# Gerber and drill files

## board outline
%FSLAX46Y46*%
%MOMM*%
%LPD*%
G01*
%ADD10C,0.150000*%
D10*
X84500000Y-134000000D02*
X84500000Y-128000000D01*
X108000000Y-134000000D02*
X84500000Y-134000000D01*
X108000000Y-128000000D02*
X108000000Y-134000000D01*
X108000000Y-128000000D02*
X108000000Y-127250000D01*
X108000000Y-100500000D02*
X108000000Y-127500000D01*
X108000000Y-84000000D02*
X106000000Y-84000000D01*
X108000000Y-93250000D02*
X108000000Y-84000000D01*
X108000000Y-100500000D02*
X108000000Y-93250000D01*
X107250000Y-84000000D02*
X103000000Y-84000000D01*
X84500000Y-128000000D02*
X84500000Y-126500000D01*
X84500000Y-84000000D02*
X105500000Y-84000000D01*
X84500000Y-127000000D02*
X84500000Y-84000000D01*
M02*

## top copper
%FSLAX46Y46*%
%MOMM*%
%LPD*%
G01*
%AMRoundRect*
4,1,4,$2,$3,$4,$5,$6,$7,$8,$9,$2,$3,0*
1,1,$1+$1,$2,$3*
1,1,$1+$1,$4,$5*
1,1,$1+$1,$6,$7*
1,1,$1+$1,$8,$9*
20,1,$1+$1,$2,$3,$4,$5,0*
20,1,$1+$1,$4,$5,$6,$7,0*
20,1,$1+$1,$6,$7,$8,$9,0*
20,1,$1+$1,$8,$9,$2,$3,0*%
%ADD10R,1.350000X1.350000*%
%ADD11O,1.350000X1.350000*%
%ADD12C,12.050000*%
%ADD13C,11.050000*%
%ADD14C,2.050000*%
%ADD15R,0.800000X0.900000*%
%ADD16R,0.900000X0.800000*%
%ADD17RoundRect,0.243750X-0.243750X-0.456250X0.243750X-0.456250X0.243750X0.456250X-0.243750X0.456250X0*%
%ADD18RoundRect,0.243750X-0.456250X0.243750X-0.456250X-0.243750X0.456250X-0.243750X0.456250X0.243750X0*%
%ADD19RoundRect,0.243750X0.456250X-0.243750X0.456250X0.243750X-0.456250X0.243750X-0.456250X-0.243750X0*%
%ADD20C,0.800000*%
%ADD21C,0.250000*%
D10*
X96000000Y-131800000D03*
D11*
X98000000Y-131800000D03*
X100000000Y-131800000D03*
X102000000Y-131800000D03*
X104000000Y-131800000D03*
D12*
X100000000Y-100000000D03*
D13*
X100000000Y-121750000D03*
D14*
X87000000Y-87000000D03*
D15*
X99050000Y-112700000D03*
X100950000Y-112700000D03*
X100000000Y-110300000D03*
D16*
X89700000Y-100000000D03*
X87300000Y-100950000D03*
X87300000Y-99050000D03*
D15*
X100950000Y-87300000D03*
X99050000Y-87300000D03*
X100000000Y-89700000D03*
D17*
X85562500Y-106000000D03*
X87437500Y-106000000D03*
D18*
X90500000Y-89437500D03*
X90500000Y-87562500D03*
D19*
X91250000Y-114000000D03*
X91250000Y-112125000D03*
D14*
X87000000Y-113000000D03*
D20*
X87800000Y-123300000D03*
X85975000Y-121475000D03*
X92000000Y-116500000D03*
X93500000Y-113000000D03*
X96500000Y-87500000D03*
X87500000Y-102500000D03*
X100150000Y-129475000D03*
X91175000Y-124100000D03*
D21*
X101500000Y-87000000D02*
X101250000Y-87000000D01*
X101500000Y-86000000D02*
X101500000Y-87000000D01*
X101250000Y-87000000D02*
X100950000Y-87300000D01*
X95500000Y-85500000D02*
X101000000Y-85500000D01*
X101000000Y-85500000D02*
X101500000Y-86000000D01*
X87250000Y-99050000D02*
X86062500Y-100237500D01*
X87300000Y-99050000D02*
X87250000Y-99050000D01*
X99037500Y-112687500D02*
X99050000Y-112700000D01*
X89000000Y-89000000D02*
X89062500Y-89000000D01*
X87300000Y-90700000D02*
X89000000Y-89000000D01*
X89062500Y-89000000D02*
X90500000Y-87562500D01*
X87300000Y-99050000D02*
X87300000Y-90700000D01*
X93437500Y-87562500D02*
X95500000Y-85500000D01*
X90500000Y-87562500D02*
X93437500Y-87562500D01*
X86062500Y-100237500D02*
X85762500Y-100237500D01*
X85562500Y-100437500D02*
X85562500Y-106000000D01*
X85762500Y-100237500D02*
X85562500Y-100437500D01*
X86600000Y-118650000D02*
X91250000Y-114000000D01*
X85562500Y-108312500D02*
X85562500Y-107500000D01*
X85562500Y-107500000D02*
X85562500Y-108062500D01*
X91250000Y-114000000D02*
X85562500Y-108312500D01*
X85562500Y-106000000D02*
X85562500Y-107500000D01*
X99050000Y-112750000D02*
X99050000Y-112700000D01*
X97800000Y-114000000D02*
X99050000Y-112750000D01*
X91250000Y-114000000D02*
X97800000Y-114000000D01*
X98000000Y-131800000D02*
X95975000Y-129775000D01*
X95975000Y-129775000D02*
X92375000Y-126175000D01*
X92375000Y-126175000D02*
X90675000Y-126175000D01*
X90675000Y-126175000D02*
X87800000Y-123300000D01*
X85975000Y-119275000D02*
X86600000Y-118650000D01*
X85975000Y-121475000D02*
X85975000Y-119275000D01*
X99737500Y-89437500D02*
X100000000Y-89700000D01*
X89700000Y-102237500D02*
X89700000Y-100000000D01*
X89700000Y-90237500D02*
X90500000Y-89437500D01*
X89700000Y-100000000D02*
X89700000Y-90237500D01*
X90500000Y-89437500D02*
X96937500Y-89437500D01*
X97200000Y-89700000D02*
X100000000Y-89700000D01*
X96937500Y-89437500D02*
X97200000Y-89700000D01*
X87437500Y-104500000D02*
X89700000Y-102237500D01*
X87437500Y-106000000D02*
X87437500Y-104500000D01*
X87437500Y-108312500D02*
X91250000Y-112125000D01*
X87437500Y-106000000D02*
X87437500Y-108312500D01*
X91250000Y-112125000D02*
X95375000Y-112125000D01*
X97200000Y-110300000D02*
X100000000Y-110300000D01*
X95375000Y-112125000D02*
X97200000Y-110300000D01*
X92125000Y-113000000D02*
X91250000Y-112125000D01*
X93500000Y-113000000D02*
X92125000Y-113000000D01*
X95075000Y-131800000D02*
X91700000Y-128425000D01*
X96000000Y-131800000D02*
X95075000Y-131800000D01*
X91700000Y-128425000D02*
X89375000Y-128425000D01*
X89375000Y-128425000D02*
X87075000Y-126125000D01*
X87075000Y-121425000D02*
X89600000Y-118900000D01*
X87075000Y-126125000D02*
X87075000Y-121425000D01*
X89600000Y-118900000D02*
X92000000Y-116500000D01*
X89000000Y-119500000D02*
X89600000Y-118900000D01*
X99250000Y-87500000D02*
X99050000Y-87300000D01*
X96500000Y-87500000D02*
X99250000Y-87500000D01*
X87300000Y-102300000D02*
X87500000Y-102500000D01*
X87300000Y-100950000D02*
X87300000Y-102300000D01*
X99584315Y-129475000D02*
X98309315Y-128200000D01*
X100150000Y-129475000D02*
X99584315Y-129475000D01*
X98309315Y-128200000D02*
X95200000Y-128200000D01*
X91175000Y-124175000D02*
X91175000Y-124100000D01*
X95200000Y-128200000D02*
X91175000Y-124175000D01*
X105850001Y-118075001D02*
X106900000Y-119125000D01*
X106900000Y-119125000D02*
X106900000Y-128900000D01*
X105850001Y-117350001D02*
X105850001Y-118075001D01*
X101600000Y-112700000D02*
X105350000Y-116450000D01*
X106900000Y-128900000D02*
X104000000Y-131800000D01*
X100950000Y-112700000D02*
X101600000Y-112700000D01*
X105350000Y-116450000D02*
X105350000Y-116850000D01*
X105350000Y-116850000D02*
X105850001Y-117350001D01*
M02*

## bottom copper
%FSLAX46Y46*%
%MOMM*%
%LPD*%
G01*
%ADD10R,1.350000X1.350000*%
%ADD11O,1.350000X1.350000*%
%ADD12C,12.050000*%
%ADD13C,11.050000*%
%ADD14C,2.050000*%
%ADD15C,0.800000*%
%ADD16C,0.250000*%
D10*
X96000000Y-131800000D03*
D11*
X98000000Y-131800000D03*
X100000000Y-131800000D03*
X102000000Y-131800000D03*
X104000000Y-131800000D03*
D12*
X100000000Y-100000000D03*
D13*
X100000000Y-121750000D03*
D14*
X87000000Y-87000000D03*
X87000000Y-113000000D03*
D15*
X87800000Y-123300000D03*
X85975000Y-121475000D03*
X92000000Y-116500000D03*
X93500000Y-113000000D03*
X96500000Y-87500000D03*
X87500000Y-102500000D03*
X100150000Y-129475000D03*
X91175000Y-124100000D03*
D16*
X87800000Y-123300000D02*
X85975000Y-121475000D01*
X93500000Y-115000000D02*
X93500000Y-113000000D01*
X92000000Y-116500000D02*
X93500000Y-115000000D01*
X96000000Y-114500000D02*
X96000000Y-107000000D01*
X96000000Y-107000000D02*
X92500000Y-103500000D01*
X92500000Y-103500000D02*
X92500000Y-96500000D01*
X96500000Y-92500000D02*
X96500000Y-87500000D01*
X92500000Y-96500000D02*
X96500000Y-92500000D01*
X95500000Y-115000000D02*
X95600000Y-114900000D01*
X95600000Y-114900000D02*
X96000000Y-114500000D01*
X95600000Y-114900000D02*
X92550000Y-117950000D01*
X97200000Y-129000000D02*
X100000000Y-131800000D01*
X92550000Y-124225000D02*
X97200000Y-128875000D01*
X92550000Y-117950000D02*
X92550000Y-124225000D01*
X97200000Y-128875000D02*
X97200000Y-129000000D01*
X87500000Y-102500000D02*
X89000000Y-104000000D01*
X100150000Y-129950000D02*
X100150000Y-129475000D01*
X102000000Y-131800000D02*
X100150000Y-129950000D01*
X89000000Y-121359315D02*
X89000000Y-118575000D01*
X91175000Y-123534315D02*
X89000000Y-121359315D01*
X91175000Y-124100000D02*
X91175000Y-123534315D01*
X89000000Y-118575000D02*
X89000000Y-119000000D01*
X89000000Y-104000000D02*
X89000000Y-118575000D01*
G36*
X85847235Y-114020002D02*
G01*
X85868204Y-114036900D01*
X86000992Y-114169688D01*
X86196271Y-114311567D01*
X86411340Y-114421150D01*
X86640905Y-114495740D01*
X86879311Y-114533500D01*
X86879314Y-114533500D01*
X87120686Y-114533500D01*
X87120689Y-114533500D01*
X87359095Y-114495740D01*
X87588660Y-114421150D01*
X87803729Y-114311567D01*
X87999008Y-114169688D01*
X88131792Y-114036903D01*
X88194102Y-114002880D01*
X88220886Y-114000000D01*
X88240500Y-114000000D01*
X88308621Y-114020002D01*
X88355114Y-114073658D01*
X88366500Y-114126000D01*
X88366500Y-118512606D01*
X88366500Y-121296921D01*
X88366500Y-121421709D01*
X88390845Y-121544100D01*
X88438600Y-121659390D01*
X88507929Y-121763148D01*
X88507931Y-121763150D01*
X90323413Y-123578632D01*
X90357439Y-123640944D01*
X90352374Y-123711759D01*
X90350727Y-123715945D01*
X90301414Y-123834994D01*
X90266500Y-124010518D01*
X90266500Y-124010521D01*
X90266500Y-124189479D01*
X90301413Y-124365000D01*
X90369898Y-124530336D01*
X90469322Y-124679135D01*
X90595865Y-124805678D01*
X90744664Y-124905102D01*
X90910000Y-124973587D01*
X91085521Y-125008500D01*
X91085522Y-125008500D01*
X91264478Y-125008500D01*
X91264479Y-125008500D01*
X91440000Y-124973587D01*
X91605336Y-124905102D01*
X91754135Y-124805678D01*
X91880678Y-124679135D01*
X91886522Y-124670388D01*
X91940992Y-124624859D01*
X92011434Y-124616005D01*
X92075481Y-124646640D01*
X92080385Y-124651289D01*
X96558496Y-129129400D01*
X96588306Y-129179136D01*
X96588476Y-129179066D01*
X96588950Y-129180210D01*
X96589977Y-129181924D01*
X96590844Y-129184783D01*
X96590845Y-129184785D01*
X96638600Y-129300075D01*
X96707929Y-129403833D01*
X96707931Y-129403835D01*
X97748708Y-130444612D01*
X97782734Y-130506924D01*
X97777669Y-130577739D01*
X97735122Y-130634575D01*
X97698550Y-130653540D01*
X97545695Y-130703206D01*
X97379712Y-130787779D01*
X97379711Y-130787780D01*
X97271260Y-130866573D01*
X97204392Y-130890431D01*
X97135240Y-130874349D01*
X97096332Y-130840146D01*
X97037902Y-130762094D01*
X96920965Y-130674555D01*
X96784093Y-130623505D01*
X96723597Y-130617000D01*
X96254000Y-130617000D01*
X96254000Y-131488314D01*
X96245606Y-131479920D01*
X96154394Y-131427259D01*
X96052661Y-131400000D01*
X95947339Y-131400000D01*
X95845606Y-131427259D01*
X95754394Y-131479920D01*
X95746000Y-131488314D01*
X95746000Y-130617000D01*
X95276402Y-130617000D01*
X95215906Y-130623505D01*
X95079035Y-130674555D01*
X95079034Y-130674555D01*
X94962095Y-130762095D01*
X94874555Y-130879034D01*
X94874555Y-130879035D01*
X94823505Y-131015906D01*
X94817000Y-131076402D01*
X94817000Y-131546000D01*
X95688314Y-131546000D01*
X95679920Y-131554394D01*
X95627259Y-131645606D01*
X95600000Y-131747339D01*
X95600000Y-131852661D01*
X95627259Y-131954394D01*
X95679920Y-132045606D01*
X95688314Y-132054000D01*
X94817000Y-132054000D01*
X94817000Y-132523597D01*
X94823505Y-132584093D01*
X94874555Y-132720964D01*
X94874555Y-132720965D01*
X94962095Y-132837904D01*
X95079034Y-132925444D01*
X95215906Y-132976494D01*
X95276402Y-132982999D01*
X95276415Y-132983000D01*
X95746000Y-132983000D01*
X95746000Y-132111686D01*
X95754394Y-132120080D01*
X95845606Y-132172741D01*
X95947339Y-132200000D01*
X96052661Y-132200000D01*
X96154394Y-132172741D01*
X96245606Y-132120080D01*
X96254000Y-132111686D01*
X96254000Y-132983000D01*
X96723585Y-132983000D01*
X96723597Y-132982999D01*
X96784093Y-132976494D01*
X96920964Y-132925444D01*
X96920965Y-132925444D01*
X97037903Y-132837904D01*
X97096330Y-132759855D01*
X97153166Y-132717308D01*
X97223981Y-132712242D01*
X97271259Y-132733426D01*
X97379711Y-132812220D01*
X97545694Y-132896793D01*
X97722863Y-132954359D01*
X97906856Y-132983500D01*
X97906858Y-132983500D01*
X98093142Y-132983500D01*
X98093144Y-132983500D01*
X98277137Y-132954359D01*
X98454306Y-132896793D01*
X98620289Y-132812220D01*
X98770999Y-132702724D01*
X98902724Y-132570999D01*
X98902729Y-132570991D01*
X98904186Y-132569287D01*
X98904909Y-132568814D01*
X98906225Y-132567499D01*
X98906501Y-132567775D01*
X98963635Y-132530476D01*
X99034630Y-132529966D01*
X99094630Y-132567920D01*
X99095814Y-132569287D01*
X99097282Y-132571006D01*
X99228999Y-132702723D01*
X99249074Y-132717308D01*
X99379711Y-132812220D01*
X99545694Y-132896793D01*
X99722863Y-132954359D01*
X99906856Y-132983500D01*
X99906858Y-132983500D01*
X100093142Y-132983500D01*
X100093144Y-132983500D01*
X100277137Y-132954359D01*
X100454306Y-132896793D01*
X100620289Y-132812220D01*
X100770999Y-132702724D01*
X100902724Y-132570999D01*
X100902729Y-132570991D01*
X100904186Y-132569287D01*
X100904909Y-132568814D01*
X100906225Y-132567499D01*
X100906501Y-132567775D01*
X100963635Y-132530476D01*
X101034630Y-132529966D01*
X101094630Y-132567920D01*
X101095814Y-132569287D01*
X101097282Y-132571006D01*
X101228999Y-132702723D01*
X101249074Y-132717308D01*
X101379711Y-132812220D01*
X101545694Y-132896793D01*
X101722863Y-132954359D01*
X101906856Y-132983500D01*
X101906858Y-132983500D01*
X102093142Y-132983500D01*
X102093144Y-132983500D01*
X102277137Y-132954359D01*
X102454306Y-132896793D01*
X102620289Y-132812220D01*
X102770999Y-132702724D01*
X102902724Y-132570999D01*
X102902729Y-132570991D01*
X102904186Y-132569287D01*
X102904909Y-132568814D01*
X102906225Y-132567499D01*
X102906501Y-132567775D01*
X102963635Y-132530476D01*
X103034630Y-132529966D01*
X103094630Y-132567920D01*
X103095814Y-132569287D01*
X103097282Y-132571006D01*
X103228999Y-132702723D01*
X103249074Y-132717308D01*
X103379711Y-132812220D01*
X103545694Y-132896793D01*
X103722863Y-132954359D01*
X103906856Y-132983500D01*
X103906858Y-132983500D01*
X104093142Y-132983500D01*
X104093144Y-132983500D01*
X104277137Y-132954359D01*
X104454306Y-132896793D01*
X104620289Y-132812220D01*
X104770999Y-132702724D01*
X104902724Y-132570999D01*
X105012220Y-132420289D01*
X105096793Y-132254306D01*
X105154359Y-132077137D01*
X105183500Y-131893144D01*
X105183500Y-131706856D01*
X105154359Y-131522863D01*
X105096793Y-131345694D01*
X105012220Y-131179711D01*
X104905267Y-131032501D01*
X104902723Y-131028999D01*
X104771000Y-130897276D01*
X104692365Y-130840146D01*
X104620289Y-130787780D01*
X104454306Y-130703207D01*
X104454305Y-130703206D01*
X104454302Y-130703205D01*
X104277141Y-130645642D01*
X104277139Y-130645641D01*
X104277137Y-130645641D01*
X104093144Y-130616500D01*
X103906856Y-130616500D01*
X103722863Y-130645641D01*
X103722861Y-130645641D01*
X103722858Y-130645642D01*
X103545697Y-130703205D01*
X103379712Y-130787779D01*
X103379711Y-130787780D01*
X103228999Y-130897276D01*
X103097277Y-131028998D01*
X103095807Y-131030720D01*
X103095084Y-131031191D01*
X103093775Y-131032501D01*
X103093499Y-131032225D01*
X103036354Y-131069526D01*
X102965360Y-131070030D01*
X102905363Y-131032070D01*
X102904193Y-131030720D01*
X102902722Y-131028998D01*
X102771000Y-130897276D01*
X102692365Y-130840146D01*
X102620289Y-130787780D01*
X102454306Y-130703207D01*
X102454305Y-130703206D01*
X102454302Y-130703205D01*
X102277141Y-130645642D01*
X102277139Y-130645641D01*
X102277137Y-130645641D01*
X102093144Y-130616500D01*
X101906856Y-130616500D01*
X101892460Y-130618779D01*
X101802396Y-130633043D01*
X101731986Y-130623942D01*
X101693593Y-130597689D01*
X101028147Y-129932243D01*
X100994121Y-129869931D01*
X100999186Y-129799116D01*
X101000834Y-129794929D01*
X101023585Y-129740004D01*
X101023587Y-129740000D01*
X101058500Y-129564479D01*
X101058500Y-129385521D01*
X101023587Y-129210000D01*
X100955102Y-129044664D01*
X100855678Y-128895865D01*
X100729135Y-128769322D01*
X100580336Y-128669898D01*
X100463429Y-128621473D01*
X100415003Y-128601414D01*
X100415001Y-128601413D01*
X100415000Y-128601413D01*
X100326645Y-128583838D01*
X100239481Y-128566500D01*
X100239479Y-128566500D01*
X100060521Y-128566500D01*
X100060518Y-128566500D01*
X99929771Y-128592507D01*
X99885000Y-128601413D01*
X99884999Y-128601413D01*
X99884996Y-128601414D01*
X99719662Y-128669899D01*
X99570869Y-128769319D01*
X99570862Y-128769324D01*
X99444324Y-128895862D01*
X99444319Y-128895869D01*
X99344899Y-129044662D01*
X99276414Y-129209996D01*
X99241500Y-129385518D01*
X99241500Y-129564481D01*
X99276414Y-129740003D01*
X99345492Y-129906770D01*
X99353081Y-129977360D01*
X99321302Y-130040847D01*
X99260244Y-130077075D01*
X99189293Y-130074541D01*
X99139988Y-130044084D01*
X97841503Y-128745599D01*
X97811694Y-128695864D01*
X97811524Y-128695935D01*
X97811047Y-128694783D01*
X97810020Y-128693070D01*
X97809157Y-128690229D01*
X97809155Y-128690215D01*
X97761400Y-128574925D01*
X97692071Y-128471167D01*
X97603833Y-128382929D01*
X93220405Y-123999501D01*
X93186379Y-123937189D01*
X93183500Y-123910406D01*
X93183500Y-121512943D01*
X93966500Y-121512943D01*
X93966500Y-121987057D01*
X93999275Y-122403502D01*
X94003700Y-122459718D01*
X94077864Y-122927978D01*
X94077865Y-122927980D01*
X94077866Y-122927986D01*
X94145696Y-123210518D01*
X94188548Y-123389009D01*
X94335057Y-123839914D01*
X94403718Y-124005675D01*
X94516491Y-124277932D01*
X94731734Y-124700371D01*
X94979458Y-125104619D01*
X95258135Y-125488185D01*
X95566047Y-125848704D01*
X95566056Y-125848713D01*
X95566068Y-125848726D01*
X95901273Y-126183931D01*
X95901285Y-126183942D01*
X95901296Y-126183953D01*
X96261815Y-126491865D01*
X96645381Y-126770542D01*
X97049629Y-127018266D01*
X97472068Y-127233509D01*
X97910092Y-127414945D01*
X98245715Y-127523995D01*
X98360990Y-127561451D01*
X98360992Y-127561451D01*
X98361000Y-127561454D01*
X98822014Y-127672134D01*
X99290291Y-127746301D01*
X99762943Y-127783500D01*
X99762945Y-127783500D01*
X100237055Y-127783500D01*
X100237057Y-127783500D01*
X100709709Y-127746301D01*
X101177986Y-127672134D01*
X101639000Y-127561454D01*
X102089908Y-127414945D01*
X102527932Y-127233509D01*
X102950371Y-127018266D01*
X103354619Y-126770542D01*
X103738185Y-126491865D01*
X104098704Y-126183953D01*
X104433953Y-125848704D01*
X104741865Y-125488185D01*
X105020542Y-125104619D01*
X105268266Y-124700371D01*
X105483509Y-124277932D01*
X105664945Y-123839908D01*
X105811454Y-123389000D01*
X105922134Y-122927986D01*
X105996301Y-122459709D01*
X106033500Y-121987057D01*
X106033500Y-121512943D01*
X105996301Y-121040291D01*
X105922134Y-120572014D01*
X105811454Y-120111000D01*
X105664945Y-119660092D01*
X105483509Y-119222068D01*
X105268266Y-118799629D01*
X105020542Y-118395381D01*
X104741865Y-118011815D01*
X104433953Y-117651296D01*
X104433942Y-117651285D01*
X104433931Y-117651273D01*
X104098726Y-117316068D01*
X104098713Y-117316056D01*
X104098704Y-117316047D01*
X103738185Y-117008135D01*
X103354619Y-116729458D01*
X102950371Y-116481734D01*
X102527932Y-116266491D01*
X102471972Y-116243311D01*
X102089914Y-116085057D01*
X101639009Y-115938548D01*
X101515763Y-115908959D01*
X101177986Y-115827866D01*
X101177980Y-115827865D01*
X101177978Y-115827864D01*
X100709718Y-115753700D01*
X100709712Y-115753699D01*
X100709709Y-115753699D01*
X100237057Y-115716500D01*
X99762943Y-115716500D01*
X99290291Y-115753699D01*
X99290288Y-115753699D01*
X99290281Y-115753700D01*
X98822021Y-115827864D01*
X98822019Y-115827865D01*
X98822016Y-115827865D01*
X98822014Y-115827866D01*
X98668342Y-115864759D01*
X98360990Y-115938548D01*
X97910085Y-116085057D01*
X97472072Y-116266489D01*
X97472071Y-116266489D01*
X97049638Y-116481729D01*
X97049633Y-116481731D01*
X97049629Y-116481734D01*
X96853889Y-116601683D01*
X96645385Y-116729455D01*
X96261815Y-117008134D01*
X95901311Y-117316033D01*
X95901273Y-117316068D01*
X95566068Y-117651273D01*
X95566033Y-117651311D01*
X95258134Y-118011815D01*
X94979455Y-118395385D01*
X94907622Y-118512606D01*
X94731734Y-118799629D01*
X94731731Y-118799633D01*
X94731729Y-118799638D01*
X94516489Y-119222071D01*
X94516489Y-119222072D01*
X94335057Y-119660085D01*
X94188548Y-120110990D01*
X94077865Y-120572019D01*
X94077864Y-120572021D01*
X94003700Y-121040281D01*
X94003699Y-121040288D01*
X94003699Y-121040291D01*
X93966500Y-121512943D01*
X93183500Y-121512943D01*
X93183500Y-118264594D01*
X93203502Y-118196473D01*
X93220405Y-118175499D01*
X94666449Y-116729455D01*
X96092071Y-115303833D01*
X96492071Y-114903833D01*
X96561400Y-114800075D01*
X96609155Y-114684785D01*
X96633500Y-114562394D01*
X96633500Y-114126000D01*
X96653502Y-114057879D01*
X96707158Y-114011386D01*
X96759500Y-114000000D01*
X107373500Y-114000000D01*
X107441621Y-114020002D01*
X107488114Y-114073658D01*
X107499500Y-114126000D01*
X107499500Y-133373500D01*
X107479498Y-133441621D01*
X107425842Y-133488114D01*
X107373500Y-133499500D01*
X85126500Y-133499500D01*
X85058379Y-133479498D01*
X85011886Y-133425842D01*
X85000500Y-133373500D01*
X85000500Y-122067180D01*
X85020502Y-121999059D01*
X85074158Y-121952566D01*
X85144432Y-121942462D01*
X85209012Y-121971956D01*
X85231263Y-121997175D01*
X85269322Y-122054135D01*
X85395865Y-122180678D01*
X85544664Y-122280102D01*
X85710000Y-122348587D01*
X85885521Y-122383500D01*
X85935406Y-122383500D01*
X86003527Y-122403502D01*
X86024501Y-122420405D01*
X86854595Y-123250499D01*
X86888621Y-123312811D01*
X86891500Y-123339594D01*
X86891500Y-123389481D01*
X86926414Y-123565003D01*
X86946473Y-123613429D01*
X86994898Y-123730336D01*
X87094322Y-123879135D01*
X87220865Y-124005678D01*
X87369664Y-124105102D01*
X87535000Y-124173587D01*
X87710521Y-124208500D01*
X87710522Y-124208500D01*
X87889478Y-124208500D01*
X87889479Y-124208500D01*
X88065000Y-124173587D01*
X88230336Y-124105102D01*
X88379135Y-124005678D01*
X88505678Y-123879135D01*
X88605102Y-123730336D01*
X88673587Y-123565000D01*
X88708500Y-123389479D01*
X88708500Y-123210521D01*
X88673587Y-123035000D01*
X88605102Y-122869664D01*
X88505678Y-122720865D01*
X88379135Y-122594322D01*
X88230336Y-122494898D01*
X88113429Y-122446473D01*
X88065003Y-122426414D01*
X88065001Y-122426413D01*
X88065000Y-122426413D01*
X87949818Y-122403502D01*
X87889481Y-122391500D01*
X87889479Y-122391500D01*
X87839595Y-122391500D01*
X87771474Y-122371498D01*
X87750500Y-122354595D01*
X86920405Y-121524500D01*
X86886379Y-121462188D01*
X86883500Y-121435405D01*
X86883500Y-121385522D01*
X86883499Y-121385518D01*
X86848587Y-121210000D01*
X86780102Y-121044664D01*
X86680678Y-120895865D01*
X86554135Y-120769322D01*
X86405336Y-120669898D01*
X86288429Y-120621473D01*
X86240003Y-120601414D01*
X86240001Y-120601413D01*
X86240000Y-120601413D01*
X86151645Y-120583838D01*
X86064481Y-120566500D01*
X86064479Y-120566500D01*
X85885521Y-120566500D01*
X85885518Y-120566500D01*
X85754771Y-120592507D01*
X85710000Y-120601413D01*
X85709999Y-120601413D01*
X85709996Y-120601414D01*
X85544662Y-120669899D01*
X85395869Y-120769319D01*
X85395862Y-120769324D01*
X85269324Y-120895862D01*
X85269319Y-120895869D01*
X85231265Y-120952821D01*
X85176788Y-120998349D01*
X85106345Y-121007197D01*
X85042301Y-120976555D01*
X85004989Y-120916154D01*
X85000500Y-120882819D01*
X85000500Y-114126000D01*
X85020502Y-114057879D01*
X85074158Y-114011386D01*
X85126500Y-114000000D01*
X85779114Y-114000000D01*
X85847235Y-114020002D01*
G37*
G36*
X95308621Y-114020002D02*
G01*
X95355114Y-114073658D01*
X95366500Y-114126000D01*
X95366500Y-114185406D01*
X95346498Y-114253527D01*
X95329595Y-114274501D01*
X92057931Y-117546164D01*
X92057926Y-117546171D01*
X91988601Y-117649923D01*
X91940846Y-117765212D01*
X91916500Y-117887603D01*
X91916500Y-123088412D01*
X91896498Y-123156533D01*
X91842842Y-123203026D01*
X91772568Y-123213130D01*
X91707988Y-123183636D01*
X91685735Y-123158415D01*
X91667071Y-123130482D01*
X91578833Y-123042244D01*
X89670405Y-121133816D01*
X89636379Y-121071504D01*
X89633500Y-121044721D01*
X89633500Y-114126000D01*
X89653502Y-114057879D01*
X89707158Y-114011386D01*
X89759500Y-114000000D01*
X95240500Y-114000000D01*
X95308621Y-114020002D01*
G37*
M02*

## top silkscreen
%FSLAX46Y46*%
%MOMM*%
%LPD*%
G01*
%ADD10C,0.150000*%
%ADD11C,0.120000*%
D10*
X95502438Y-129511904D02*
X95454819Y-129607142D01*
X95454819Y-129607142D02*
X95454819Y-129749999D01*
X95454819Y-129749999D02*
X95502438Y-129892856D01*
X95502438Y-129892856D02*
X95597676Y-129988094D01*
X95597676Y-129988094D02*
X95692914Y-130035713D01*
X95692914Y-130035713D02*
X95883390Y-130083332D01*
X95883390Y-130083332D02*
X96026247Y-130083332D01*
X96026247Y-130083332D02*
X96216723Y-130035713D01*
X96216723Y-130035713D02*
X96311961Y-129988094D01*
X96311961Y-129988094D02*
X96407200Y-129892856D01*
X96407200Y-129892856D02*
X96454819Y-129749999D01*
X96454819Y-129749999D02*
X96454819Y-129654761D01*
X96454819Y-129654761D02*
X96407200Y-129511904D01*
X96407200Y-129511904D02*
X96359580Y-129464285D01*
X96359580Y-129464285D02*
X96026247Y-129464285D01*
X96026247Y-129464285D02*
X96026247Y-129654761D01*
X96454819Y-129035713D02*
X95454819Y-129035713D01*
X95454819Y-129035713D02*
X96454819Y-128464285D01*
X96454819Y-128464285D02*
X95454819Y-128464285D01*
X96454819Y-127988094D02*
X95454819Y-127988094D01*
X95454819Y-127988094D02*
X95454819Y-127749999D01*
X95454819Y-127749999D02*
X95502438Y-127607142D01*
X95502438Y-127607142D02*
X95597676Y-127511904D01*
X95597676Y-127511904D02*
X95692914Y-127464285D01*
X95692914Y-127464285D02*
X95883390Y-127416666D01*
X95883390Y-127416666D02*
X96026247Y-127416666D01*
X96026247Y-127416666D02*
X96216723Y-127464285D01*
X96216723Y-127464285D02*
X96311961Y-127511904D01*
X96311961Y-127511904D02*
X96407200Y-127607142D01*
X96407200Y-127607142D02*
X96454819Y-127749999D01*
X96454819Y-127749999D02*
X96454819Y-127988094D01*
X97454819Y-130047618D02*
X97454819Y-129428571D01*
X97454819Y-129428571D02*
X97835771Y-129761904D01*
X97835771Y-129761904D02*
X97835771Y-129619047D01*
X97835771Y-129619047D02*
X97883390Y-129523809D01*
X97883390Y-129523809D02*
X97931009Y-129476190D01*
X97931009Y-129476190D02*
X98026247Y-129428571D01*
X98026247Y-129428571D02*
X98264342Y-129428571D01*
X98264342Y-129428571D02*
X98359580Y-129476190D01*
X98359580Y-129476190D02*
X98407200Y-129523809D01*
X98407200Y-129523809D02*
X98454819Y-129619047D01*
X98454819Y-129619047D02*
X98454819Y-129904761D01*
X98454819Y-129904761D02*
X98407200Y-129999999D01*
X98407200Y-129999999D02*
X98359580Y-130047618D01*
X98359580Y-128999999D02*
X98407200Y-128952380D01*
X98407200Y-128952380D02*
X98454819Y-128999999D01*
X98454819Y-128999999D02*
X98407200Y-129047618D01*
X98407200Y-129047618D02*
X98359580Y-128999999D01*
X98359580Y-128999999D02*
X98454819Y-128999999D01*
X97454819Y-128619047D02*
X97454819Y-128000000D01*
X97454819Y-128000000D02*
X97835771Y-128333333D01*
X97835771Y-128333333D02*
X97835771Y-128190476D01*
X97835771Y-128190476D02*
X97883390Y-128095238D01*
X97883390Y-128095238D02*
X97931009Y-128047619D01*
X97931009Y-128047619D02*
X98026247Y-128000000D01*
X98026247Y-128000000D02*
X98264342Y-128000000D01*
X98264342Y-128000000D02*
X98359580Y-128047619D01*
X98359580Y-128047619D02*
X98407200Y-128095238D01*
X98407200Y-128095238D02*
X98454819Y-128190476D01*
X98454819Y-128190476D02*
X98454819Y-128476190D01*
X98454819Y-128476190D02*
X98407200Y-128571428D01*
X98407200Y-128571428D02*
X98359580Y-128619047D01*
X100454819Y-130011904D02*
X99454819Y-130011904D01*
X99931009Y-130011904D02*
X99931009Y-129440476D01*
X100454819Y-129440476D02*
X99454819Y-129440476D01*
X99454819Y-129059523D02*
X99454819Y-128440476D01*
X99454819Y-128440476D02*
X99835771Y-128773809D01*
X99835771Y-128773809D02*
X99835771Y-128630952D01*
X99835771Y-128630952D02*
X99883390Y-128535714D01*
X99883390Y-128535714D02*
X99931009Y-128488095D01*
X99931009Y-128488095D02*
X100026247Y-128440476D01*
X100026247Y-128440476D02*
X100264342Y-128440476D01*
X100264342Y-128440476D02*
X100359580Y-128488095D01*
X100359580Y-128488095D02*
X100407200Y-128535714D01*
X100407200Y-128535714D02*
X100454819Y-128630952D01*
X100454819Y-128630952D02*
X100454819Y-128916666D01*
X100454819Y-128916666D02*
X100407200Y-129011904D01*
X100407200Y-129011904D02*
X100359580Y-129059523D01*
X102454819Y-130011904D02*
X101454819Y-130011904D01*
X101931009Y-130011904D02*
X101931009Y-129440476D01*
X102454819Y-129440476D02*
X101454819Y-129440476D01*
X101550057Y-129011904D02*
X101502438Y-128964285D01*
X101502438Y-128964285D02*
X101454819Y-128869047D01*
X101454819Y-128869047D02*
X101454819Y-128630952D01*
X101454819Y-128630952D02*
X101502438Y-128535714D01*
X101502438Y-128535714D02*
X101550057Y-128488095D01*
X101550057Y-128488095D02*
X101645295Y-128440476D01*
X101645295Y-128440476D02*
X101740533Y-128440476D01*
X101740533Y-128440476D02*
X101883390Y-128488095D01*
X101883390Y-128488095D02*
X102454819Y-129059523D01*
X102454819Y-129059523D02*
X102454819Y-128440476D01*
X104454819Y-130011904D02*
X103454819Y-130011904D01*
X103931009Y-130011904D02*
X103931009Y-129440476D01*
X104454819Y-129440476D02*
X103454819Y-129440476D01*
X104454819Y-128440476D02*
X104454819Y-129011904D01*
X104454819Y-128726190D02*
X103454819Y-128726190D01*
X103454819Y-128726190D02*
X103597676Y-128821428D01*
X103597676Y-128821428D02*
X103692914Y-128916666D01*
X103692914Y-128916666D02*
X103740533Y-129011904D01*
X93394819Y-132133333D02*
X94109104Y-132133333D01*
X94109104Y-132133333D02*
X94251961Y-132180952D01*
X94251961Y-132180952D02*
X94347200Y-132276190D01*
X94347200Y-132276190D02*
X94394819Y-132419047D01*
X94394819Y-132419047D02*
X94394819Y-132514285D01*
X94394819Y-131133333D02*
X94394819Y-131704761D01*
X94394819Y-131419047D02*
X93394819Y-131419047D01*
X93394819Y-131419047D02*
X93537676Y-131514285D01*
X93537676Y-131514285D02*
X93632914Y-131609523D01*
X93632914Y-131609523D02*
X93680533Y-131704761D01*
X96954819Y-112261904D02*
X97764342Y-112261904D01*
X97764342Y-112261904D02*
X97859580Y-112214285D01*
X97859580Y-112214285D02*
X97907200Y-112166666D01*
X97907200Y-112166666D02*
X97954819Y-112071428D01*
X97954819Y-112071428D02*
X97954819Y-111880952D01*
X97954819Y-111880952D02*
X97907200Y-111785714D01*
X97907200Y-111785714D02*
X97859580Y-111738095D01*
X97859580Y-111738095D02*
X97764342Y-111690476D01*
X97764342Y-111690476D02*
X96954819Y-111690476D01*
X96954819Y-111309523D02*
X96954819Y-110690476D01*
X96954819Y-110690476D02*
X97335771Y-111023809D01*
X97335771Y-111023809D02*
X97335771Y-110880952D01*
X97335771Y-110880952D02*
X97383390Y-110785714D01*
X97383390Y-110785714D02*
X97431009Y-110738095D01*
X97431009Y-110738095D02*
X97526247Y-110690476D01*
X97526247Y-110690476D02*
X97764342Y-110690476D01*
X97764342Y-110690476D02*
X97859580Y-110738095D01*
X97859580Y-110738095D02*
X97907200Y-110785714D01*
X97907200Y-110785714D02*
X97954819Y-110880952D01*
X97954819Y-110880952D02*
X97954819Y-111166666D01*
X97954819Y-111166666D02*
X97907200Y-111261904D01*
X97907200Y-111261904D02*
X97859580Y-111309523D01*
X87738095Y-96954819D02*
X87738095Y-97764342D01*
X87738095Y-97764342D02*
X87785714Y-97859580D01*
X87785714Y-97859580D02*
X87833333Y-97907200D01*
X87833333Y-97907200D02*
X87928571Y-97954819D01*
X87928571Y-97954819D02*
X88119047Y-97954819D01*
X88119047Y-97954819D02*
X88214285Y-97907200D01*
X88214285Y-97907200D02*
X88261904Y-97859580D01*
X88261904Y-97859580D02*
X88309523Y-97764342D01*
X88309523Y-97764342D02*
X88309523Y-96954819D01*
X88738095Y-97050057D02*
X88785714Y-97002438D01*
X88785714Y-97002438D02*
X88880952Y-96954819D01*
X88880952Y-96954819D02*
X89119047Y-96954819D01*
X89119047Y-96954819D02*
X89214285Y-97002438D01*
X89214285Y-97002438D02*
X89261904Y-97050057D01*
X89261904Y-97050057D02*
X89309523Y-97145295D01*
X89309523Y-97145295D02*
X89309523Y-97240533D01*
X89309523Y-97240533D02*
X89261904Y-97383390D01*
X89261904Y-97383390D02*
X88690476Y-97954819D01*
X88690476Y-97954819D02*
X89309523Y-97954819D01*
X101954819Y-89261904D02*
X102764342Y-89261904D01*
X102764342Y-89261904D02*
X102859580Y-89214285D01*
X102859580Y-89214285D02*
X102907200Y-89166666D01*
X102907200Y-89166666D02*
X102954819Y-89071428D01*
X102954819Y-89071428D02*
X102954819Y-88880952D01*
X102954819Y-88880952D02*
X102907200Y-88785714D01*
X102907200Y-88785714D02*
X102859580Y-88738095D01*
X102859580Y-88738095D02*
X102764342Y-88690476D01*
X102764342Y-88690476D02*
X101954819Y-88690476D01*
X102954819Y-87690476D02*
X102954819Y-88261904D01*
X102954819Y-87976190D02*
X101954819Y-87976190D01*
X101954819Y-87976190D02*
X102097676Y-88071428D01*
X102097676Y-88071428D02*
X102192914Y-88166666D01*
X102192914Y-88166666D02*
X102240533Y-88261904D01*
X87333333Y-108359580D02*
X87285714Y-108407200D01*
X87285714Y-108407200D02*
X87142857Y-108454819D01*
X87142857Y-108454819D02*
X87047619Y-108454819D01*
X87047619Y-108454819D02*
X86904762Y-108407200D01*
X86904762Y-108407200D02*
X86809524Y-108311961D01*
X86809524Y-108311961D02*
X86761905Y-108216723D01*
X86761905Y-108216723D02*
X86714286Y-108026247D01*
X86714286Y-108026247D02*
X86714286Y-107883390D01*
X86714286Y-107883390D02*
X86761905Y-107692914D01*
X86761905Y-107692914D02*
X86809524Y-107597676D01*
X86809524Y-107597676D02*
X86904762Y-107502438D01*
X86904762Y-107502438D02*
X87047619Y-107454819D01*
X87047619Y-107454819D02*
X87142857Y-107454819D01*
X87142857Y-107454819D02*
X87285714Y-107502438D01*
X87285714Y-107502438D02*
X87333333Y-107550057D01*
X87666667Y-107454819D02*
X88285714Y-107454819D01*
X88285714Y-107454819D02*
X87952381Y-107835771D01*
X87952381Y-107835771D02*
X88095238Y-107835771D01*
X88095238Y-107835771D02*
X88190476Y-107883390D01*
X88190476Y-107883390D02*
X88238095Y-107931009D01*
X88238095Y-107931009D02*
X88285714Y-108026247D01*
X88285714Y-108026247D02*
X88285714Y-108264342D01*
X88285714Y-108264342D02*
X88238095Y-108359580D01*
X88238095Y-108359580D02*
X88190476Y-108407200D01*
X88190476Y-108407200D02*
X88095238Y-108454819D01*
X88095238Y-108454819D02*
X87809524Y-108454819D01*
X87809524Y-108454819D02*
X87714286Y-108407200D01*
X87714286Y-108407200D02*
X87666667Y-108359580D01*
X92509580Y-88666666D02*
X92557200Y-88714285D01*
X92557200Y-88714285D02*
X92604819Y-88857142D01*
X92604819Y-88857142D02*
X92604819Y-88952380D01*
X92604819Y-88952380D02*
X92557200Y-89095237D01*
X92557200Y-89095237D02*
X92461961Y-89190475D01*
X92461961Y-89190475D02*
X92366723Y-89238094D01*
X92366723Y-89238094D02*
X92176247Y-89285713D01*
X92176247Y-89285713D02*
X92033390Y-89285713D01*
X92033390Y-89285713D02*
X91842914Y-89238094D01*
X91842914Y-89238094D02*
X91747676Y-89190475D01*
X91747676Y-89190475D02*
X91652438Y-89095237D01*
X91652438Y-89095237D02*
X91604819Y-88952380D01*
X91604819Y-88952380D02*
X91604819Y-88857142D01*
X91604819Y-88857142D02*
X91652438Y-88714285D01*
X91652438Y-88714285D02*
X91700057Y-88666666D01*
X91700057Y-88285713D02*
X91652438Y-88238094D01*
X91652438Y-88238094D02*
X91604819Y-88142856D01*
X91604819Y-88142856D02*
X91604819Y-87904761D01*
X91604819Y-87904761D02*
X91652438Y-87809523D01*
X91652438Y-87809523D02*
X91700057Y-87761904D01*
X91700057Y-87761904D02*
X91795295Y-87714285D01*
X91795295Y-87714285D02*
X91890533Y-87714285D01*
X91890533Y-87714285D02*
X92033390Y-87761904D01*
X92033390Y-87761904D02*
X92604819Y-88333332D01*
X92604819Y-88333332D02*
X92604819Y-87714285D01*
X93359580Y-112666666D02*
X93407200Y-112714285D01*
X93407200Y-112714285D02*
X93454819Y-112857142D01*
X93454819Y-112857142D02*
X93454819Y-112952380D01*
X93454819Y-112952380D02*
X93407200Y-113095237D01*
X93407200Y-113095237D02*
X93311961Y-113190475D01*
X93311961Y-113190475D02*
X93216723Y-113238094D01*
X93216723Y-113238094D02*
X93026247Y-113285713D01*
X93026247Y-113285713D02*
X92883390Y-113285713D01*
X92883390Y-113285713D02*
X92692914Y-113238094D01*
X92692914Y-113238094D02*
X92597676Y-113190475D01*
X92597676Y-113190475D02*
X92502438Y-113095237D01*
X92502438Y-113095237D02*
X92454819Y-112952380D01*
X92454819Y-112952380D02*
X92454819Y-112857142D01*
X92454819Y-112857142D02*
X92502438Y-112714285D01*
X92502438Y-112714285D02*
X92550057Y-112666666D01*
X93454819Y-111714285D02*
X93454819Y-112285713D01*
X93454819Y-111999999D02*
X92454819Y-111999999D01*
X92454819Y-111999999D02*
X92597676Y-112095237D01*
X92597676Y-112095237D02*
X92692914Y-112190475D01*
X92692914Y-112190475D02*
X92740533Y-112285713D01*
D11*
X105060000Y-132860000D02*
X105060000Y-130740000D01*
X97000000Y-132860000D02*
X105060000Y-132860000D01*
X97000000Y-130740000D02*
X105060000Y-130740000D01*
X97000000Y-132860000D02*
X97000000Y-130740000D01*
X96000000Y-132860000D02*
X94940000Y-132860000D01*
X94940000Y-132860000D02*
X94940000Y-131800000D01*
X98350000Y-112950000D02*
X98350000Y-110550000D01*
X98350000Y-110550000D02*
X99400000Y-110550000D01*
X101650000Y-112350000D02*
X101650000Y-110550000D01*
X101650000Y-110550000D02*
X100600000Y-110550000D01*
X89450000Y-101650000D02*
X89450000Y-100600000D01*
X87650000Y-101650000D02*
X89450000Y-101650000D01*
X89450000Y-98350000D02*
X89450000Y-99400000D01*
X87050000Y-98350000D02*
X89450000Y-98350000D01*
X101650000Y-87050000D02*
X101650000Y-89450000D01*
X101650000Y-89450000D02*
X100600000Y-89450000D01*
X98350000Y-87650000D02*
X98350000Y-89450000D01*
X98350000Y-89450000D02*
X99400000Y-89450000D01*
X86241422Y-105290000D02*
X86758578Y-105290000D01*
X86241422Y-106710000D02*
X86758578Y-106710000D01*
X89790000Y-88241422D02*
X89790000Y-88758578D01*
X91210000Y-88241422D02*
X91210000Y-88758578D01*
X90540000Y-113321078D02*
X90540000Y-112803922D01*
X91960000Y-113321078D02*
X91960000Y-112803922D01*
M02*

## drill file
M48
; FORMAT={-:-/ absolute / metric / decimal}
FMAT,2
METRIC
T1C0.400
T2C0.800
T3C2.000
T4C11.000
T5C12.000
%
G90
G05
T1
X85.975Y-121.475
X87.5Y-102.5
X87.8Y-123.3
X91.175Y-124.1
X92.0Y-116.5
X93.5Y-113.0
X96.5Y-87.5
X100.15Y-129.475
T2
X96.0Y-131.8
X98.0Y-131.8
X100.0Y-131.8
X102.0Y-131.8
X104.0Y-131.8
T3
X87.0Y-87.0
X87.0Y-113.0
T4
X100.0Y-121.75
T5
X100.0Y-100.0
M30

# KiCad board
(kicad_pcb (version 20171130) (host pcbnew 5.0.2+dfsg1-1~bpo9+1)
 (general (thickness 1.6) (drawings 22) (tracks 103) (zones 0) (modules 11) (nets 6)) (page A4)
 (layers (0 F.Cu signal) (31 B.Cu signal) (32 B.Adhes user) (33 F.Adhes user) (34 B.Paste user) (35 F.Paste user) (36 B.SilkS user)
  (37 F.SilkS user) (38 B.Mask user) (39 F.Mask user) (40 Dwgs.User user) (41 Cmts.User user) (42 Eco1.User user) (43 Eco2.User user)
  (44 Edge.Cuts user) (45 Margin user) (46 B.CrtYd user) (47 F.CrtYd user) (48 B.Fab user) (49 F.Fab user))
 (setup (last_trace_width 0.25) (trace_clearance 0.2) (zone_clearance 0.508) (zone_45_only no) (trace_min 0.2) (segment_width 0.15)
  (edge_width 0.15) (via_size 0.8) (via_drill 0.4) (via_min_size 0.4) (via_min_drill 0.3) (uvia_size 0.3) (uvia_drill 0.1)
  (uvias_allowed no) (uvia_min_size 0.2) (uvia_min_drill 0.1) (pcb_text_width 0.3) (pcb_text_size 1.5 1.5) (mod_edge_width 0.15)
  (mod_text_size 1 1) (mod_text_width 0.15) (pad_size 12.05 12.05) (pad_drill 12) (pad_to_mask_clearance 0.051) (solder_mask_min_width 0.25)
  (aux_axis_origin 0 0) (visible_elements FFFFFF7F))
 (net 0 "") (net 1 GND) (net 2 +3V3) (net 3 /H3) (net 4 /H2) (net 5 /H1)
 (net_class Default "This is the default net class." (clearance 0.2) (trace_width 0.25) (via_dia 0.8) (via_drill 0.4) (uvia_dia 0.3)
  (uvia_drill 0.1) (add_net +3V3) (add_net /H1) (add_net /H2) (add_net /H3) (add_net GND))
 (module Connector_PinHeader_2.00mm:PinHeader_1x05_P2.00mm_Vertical (layer F.Cu) (at 96 131.8 90)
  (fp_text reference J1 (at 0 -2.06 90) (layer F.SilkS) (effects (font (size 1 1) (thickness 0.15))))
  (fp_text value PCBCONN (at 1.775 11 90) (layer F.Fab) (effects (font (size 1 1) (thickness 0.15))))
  (fp_line (start -1.06 9.06) (end 1.06 9.06) (layer F.SilkS) (width 0.12))
  (fp_line (start -1.06 1) (end -1.06 9.06) (layer F.SilkS) (width 0.12))
  (fp_line (start 1.06 1) (end 1.06 9.06) (layer F.SilkS) (width 0.12))
  (fp_line (start -1.06 1) (end 1.06 1) (layer F.SilkS) (width 0.12))
  (fp_line (start -1.06 0) (end -1.06 -1.06) (layer F.SilkS) (width 0.12))
  (fp_line (start -1.06 -1.06) (end 0 -1.06) (layer F.SilkS) (width 0.12))
  (pad 1 thru_hole rect (at 0 0 90) (size 1.35 1.35) (drill 0.8) (layers *.Cu *.Mask) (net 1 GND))
  (pad 2 thru_hole oval (at 0 2 90) (size 1.35 1.35) (drill 0.8) (layers *.Cu *.Mask) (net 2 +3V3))
  (pad 3 thru_hole oval (at 0 4 90) (size 1.35 1.35) (drill 0.8) (layers *.Cu *.Mask) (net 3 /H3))
  (pad 4 thru_hole oval (at 0 6 90) (size 1.35 1.35) (drill 0.8) (layers *.Cu *.Mask) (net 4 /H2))
  (pad 5 thru_hole oval (at 0 8 90) (size 1.35 1.35) (drill 0.8) (layers *.Cu *.Mask) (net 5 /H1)))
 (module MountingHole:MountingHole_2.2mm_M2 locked (layer F.Cu) (at 100 100)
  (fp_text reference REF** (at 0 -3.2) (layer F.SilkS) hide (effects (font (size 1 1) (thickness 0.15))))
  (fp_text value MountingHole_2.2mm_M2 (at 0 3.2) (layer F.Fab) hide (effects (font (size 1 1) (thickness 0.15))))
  (pad "" np_thru_hole circle (at 0 0) (size 12.05 12.05) (drill 12) (layers *.Cu *.Mask)))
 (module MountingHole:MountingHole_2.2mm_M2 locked (layer F.Cu) (at 100 121.75)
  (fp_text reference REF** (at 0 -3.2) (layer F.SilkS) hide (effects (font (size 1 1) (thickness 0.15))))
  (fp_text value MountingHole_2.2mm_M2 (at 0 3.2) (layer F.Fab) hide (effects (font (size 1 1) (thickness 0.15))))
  (pad "" np_thru_hole circle (at 0 0) (size 11.05 11.05) (drill 11) (layers *.Cu *.Mask)))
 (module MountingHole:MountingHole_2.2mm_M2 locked (layer F.Cu) (at 87 87)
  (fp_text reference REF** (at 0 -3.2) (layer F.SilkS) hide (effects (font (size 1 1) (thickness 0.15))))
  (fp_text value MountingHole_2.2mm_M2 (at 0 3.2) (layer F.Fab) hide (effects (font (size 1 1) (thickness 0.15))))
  (pad "" np_thru_hole circle (at 0 0) (size 2.05 2.05) (drill 2) (layers *.Cu *.Mask)))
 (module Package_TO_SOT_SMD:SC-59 (layer F.Cu) (at 100 111.5 90)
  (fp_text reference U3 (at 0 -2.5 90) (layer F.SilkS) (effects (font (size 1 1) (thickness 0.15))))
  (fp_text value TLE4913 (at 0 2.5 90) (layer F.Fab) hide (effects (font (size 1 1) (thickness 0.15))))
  (fp_line (start -1.45 -1.65) (end 0.95 -1.65) (layer F.SilkS) (width 0.12))
  (fp_line (start 0.95 -1.65) (end 0.95 -0.6) (layer F.SilkS) (width 0.12))
  (fp_line (start -0.85 1.65) (end 0.95 1.65) (layer F.SilkS) (width 0.12))
  (fp_line (start 0.95 1.65) (end 0.95 0.6) (layer F.SilkS) (width 0.12))
  (pad 1 smd rect (at -1.2 -0.95 90) (size 0.9 0.8) (layers F.Cu F.Paste F.Mask) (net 2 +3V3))
  (pad 2 smd rect (at -1.2 0.95 90) (size 0.9 0.8) (layers F.Cu F.Paste F.Mask) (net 5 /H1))
  (pad 3 smd rect (at 1.2 0 90) (size 0.9 0.8) (layers F.Cu F.Paste F.Mask) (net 1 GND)))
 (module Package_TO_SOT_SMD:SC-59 (layer F.Cu) (at 88.5 100)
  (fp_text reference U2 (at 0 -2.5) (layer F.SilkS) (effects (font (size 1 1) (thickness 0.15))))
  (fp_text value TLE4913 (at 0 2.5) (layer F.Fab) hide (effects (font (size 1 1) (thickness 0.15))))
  (fp_line (start 0.95 1.65) (end 0.95 0.6) (layer F.SilkS) (width 0.12))
  (fp_line (start -0.85 1.65) (end 0.95 1.65) (layer F.SilkS) (width 0.12))
  (fp_line (start 0.95 -1.65) (end 0.95 -0.6) (layer F.SilkS) (width 0.12))
  (fp_line (start -1.45 -1.65) (end 0.95 -1.65) (layer F.SilkS) (width 0.12))
  (pad 3 smd rect (at 1.2 0) (size 0.9 0.8) (layers F.Cu F.Paste F.Mask) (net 1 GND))
  (pad 2 smd rect (at -1.2 0.95) (size 0.9 0.8) (layers F.Cu F.Paste F.Mask) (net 4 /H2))
  (pad 1 smd rect (at -1.2 -0.95) (size 0.9 0.8) (layers F.Cu F.Paste F.Mask) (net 2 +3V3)))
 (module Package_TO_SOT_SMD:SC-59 (layer F.Cu) (at 100 88.5 270)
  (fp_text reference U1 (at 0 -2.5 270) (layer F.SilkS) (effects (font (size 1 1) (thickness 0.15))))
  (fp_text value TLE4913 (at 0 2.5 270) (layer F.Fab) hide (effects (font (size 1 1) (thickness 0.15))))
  (fp_line (start -1.45 -1.65) (end 0.95 -1.65) (layer F.SilkS) (width 0.12))
  (fp_line (start 0.95 -1.65) (end 0.95 -0.6) (layer F.SilkS) (width 0.12))
  (fp_line (start -0.85 1.65) (end 0.95 1.65) (layer F.SilkS) (width 0.12))
  (fp_line (start 0.95 1.65) (end 0.95 0.6) (layer F.SilkS) (width 0.12))
  (pad 1 smd rect (at -1.2 -0.95 270) (size 0.9 0.8) (layers F.Cu F.Paste F.Mask) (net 2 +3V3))
  (pad 2 smd rect (at -1.2 0.95 270) (size 0.9 0.8) (layers F.Cu F.Paste F.Mask) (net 3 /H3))
  (pad 3 smd rect (at 1.2 0 270) (size 0.9 0.8) (layers F.Cu F.Paste F.Mask) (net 1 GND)))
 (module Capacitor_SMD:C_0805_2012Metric (layer F.Cu) (at 86.5 106)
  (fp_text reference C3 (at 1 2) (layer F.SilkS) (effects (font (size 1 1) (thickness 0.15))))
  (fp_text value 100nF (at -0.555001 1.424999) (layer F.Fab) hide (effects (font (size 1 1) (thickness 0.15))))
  (fp_line (start -0.258578 -0.71) (end 0.258578 -0.71) (layer F.SilkS) (width 0.12))
  (fp_line (start -0.258578 0.71) (end 0.258578 0.71) (layer F.SilkS) (width 0.12))
  (pad 1 smd roundrect (at -0.9375 0) (size 0.975 1.4) (layers F.Cu F.Paste F.Mask) (roundrect_rratio 0.25) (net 2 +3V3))
  (pad 2 smd roundrect (at 0.9375 0) (size 0.975 1.4) (layers F.Cu F.Paste F.Mask) (roundrect_rratio 0.25) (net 1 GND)))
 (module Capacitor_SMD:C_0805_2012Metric (layer F.Cu) (at 90.5 88.5 270)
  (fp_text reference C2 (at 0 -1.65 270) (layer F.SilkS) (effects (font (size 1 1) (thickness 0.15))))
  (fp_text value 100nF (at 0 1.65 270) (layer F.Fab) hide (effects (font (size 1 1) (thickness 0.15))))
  (fp_line (start -0.258578 0.71) (end 0.258578 0.71) (layer F.SilkS) (width 0.12))
  (fp_line (start -0.258578 -0.71) (end 0.258578 -0.71) (layer F.SilkS) (width 0.12))
  (pad 2 smd roundrect (at 0.9375 0 270) (size 0.975 1.4) (layers F.Cu F.Paste F.Mask) (roundrect_rratio 0.25) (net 1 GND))
  (pad 1 smd roundrect (at -0.9375 0 270) (size 0.975 1.4) (layers F.Cu F.Paste F.Mask) (roundrect_rratio 0.25) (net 2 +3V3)))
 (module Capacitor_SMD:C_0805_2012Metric (layer F.Cu) (at 91.25 113.0625 90)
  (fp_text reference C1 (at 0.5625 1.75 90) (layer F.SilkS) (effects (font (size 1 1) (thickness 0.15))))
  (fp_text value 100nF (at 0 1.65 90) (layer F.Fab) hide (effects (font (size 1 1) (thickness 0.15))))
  (fp_line (start -0.258578 -0.71) (end 0.258578 -0.71) (layer F.SilkS) (width 0.12))
  (fp_line (start -0.258578 0.71) (end 0.258578 0.71) (layer F.SilkS) (width 0.12))
  (pad 1 smd roundrect (at -0.9375 0 90) (size 0.975 1.4) (layers F.Cu F.Paste F.Mask) (roundrect_rratio 0.25) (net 2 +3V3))
  (pad 2 smd roundrect (at 0.9375 0 90) (size 0.975 1.4) (layers F.Cu F.Paste F.Mask) (roundrect_rratio 0.25) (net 1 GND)))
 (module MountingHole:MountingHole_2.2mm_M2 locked (layer F.Cu) (at 87 113)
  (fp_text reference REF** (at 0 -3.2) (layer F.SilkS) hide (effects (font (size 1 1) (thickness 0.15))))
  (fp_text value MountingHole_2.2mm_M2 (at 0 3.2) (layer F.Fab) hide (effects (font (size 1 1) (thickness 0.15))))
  (pad "" np_thru_hole circle (at 0 0) (size 2.05 2.05) (drill 2) (layers *.Cu *.Mask)))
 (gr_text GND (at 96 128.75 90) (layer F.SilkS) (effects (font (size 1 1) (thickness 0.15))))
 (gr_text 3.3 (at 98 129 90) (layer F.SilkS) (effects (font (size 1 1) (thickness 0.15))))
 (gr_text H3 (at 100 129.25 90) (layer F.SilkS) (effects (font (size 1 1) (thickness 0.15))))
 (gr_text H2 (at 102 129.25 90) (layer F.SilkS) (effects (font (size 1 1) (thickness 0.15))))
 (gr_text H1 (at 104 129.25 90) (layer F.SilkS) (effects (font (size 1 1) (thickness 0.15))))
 (gr_line (start 84.5 134) (end 84.5 128) (layer Edge.Cuts) (width 0.15))
 (gr_line (start 108 134) (end 84.5 134) (layer Edge.Cuts) (width 0.15))
 (gr_line (start 108 128) (end 108 134) (layer Edge.Cuts) (width 0.15))
 (gr_line (start 108 128) (end 108 127.25) (layer Edge.Cuts) (width 0.15))
 (gr_line (start 108 100.5) (end 108 127.5) (layer Edge.Cuts) (width 0.15))
 (gr_line (start 108 84) (end 106 84) (layer Edge.Cuts) (width 0.15))
 (gr_line (start 108 93.25) (end 108 84) (layer Edge.Cuts) (width 0.15))
 (gr_line (start 108 100.5) (end 108 93.25) (layer Edge.Cuts) (width 0.15))
 (gr_line (start 107.25 84) (end 103 84) (layer Edge.Cuts) (width 0.15))
 (gr_line (start 84.5 128) (end 84.5 126.5) (layer Edge.Cuts) (width 0.15))
 (gr_line (start 84.5 84) (end 105.5 84) (layer Edge.Cuts) (width 0.15))
 (gr_line (start 84.5 127) (end 84.5 84) (layer Edge.Cuts) (width 0.15))
 (segment (start 101.5 87) (end 101.25 87) (width 0.25) (layer F.Cu) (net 2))
 (segment (start 101.5 86) (end 101.5 87) (width 0.25) (layer F.Cu) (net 2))
 (segment (start 101.25 87) (end 100.95 87.3) (width 0.25) (layer F.Cu) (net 2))
 (segment (start 95.5 85.5) (end 101 85.5) (width 0.25) (layer F.Cu) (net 2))
 (segment (start 101 85.5) (end 101.5 86) (width 0.25) (layer F.Cu) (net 2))
 (segment (start 87.25 99.05) (end 86.0625 100.2375) (width 0.25) (layer F.Cu) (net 2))
 (segment (start 87.3 99.05) (end 87.25 99.05) (width 0.25) (layer F.Cu) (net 2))
 (segment (start 99.0375 112.6875) (end 99.05 112.7) (width 0.25) (layer F.Cu) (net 2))
 (segment (start 89 89) (end 89.0625 89) (width 0.25) (layer F.Cu) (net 2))
 (segment (start 87.3 90.7) (end 89 89) (width 0.25) (layer F.Cu) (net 2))
 (segment (start 89.0625 89) (end 90.5 87.5625) (width 0.25) (layer F.Cu) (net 2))
 (segment (start 87.3 99.05) (end 87.3 90.7) (width 0.25) (layer F.Cu) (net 2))
 (segment (start 93.4375 87.5625) (end 95.5 85.5) (width 0.25) (layer F.Cu) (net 2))
 (segment (start 90.5 87.5625) (end 93.4375 87.5625) (width 0.25) (layer F.Cu) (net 2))
 (segment (start 86.0625 100.2375) (end 85.7625 100.2375) (width 0.25) (layer F.Cu) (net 2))
 (segment (start 85.5625 100.4375) (end 85.5625 106) (width 0.25) (layer F.Cu) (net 2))
 (segment (start 85.7625 100.2375) (end 85.5625 100.4375) (width 0.25) (layer F.Cu) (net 2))
 (segment (start 86.6 118.65) (end 91.25 114) (width 0.25) (layer F.Cu) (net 2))
 (segment (start 85.5625 108.3125) (end 85.5625 107.5) (width 0.25) (layer F.Cu) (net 2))
 (segment (start 85.5625 107.5) (end 85.5625 108.0625) (width 0.25) (layer F.Cu) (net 2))
 (segment (start 91.25 114) (end 85.5625 108.3125) (width 0.25) (layer F.Cu) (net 2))
 (segment (start 85.5625 106) (end 85.5625 107.5) (width 0.25) (layer F.Cu) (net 2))
 (segment (start 99.05 112.75) (end 99.05 112.7) (width 0.25) (layer F.Cu) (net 2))
 (segment (start 97.8 114) (end 99.05 112.75) (width 0.25) (layer F.Cu) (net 2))
 (segment (start 91.25 114) (end 97.8 114) (width 0.25) (layer F.Cu) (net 2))
 (segment (start 98 131.8) (end 95.975 129.775) (width 0.25) (layer F.Cu) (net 2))
 (segment (start 95.975 129.775) (end 92.375 126.175) (width 0.25) (layer F.Cu) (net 2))
 (segment (start 92.375 126.175) (end 90.675 126.175) (width 0.25) (layer F.Cu) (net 2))
 (via (at 87.8 123.3) (size 0.8) (drill 0.4) (layers F.Cu B.Cu) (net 2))
 (segment (start 90.675 126.175) (end 87.8 123.3) (width 0.25) (layer F.Cu) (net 2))
 (segment (start 87.8 123.3) (end 85.975 121.475) (width 0.25) (layer B.Cu) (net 2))
 (via (at 85.975 121.475) (size 0.8) (drill 0.4) (layers F.Cu B.Cu) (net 2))
 (segment (start 85.975 119.275) (end 86.6 118.65) (width 0.25) (layer F.Cu) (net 2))
 (segment (start 85.975 121.475) (end 85.975 119.275) (width 0.25) (layer F.Cu) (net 2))
 (segment (start 99.7375 89.4375) (end 100 89.7) (width 0.25) (layer F.Cu) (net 1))
 (segment (start 89.7 102.2375) (end 89.7 100) (width 0.25) (layer F.Cu) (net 1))
 (segment (start 89.7 90.2375) (end 90.5 89.4375) (width 0.25) (layer F.Cu) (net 1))
 (segment (start 89.7 100) (end 89.7 90.2375) (width 0.25) (layer F.Cu) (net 1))
 (segment (start 90.5 89.4375) (end 96.9375 89.4375) (width 0.25) (layer F.Cu) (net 1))
 (segment (start 97.2 89.7) (end 100 89.7) (width 0.25) (layer F.Cu) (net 1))
 (segment (start 96.9375 89.4375) (end 97.2 89.7) (width 0.25) (layer F.Cu) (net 1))
 (segment (start 87.4375 104.5) (end 89.7 102.2375) (width 0.25) (layer F.Cu) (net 1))
 (segment (start 87.4375 106) (end 87.4375 104.5) (width 0.25) (layer F.Cu) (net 1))
 (segment (start 87.4375 108.3125) (end 91.25 112.125) (width 0.25) (layer F.Cu) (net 1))
 (segment (start 87.4375 106) (end 87.4375 108.3125) (width 0.25) (layer F.Cu) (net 1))
 (segment (start 91.25 112.125) (end 95.375 112.125) (width 0.25) (layer F.Cu) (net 1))
 (segment (start 97.2 110.3) (end 100 110.3) (width 0.25) (layer F.Cu) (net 1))
 (segment (start 95.375 112.125) (end 97.2 110.3) (width 0.25) (layer F.Cu) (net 1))
 (via (at 92 116.5) (size 0.8) (drill 0.4) (layers F.Cu B.Cu) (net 1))
 (via (at 93.5 113) (size 0.8) (drill 0.4) (layers F.Cu B.Cu) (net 1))
 (segment (start 93.5 115) (end 93.5 113) (width 0.25) (layer B.Cu) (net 1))
 (segment (start 92 116.5) (end 93.5 115) (width 0.25) (layer B.Cu) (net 1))
 (segment (start 92.125 113) (end 91.25 112.125) (width 0.25) (layer F.Cu) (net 1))
 (segment (start 93.5 113) (end 92.125 113) (width 0.25) (layer F.Cu) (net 1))
 (segment (start 95.075 131.8) (end 91.7 128.425) (width 0.25) (layer F.Cu) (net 1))
 (segment (start 96 131.8) (end 95.075 131.8) (width 0.25) (layer F.Cu) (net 1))
 (segment (start 91.7 128.425) (end 89.375 128.425) (width 0.25) (layer F.Cu) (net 1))
 (segment (start 89.375 128.425) (end 87.075 126.125) (width 0.25) (layer F.Cu) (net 1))
 (segment (start 87.075 121.425) (end 89.6 118.9) (width 0.25) (layer F.Cu) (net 1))
 (segment (start 87.075 126.125) (end 87.075 121.425) (width 0.25) (layer F.Cu) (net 1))
 (segment (start 89.6 118.9) (end 92 116.5) (width 0.25) (layer F.Cu) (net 1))
 (segment (start 89 119.5) (end 89.6 118.9) (width 0.25) (layer F.Cu) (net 1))
 (segment (start 96 114.5) (end 96 107) (width 0.25) (layer B.Cu) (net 3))
 (segment (start 96 107) (end 92.5 103.5) (width 0.25) (layer B.Cu) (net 3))
 (segment (start 92.5 103.5) (end 92.5 96.5) (width 0.25) (layer B.Cu) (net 3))
 (via (at 96.5 87.5) (size 0.8) (drill 0.4) (layers F.Cu B.Cu) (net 3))
 (segment (start 96.5 92.5) (end 96.5 87.5) (width 0.25) (layer B.Cu) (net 3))
 (segment (start 92.5 96.5) (end 96.5 92.5) (width 0.25) (layer B.Cu) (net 3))
 (segment (start 99.25 87.5) (end 99.05 87.3) (width 0.25) (layer F.Cu) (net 3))
 (segment (start 96.5 87.5) (end 99.25 87.5) (width 0.25) (layer F.Cu) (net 3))
 (segment (start 95.5 115) (end 95.6 114.9) (width 0.25) (layer B.Cu) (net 3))
 (segment (start 95.6 114.9) (end 96 114.5) (width 0.25) (layer B.Cu) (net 3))
 (segment (start 95.6 114.9) (end 92.55 117.95) (width 0.25) (layer B.Cu) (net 3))
 (segment (start 97.2 129) (end 100 131.8) (width 0.25) (layer B.Cu) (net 3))
 (segment (start 92.55 124.225) (end 97.2 128.875) (width 0.25) (layer B.Cu) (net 3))
 (segment (start 92.55 117.95) (end 92.55 124.225) (width 0.25) (layer B.Cu) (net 3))
 (segment (start 97.2 128.875) (end 97.2 129) (width 0.25) (layer B.Cu) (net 3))
 (via (at 87.5 102.5) (size 0.8) (drill 0.4) (layers F.Cu B.Cu) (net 4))
 (segment (start 87.3 102.3) (end 87.5 102.5) (width 0.25) (layer F.Cu) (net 4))
 (segment (start 87.3 100.95) (end 87.3 102.3) (width 0.25) (layer F.Cu) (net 4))
 (segment (start 87.5 102.5) (end 89 104) (width 0.25) (layer B.Cu) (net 4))
 (via (at 100.15 129.475) (size 0.8) (drill 0.4) (layers F.Cu B.Cu) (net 4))
 (segment (start 100.15 129.95) (end 100.15 129.475) (width 0.25) (layer B.Cu) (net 4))
 (segment (start 102 131.8) (end 100.15 129.95) (width 0.25) (layer B.Cu) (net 4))
 (segment (start 99.584315 129.475) (end 98.309315 128.2) (width 0.25) (layer F.Cu) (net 4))
 (segment (start 100.15 129.475) (end 99.584315 129.475) (width 0.25) (layer F.Cu) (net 4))
 (segment (start 98.309315 128.2) (end 95.2 128.2) (width 0.25) (layer F.Cu) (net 4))
 (via (at 91.175 124.1) (size 0.8) (drill 0.4) (layers F.Cu B.Cu) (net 4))
 (segment (start 91.175 124.175) (end 91.175 124.1) (width 0.25) (layer F.Cu) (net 4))
 (segment (start 95.2 128.2) (end 91.175 124.175) (width 0.25) (layer F.Cu) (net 4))
 (segment (start 89 121.359315) (end 89 118.575) (width 0.25) (layer B.Cu) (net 4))
 (segment (start 91.175 123.534315) (end 89 121.359315) (width 0.25) (layer B.Cu) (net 4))
 (segment (start 91.175 124.1) (end 91.175 123.534315) (width 0.25) (layer B.Cu) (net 4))
 (segment (start 89 118.575) (end 89 119) (width 0.25) (layer B.Cu) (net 4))
 (segment (start 89 104) (end 89 118.575) (width 0.25) (layer B.Cu) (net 4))
 (segment (start 105.850001 118.075001) (end 106.9 119.125) (width 0.25) (layer F.Cu) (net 5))
 (segment (start 106.9 119.125) (end 106.9 128.9) (width 0.25) (layer F.Cu) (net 5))
 (segment (start 105.850001 117.350001) (end 105.850001 118.075001) (width 0.25) (layer F.Cu) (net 5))
 (segment (start 101.6 112.7) (end 105.35 116.45) (width 0.25) (layer F.Cu) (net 5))
 (segment (start 106.9 128.9) (end 104 131.8) (width 0.25) (layer F.Cu) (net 5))
 (segment (start 100.95 112.7) (end 101.6 112.7) (width 0.25) (layer F.Cu) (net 5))
 (segment (start 105.35 116.45) (end 105.35 116.85) (width 0.25) (layer F.Cu) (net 5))
 (segment (start 105.35 116.85) (end 105.850001 117.350001) (width 0.25) (layer F.Cu) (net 5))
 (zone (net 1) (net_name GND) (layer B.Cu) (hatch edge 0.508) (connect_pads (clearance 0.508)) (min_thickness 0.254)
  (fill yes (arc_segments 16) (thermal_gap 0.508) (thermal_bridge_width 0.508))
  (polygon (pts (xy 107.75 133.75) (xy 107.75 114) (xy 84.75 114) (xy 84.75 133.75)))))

